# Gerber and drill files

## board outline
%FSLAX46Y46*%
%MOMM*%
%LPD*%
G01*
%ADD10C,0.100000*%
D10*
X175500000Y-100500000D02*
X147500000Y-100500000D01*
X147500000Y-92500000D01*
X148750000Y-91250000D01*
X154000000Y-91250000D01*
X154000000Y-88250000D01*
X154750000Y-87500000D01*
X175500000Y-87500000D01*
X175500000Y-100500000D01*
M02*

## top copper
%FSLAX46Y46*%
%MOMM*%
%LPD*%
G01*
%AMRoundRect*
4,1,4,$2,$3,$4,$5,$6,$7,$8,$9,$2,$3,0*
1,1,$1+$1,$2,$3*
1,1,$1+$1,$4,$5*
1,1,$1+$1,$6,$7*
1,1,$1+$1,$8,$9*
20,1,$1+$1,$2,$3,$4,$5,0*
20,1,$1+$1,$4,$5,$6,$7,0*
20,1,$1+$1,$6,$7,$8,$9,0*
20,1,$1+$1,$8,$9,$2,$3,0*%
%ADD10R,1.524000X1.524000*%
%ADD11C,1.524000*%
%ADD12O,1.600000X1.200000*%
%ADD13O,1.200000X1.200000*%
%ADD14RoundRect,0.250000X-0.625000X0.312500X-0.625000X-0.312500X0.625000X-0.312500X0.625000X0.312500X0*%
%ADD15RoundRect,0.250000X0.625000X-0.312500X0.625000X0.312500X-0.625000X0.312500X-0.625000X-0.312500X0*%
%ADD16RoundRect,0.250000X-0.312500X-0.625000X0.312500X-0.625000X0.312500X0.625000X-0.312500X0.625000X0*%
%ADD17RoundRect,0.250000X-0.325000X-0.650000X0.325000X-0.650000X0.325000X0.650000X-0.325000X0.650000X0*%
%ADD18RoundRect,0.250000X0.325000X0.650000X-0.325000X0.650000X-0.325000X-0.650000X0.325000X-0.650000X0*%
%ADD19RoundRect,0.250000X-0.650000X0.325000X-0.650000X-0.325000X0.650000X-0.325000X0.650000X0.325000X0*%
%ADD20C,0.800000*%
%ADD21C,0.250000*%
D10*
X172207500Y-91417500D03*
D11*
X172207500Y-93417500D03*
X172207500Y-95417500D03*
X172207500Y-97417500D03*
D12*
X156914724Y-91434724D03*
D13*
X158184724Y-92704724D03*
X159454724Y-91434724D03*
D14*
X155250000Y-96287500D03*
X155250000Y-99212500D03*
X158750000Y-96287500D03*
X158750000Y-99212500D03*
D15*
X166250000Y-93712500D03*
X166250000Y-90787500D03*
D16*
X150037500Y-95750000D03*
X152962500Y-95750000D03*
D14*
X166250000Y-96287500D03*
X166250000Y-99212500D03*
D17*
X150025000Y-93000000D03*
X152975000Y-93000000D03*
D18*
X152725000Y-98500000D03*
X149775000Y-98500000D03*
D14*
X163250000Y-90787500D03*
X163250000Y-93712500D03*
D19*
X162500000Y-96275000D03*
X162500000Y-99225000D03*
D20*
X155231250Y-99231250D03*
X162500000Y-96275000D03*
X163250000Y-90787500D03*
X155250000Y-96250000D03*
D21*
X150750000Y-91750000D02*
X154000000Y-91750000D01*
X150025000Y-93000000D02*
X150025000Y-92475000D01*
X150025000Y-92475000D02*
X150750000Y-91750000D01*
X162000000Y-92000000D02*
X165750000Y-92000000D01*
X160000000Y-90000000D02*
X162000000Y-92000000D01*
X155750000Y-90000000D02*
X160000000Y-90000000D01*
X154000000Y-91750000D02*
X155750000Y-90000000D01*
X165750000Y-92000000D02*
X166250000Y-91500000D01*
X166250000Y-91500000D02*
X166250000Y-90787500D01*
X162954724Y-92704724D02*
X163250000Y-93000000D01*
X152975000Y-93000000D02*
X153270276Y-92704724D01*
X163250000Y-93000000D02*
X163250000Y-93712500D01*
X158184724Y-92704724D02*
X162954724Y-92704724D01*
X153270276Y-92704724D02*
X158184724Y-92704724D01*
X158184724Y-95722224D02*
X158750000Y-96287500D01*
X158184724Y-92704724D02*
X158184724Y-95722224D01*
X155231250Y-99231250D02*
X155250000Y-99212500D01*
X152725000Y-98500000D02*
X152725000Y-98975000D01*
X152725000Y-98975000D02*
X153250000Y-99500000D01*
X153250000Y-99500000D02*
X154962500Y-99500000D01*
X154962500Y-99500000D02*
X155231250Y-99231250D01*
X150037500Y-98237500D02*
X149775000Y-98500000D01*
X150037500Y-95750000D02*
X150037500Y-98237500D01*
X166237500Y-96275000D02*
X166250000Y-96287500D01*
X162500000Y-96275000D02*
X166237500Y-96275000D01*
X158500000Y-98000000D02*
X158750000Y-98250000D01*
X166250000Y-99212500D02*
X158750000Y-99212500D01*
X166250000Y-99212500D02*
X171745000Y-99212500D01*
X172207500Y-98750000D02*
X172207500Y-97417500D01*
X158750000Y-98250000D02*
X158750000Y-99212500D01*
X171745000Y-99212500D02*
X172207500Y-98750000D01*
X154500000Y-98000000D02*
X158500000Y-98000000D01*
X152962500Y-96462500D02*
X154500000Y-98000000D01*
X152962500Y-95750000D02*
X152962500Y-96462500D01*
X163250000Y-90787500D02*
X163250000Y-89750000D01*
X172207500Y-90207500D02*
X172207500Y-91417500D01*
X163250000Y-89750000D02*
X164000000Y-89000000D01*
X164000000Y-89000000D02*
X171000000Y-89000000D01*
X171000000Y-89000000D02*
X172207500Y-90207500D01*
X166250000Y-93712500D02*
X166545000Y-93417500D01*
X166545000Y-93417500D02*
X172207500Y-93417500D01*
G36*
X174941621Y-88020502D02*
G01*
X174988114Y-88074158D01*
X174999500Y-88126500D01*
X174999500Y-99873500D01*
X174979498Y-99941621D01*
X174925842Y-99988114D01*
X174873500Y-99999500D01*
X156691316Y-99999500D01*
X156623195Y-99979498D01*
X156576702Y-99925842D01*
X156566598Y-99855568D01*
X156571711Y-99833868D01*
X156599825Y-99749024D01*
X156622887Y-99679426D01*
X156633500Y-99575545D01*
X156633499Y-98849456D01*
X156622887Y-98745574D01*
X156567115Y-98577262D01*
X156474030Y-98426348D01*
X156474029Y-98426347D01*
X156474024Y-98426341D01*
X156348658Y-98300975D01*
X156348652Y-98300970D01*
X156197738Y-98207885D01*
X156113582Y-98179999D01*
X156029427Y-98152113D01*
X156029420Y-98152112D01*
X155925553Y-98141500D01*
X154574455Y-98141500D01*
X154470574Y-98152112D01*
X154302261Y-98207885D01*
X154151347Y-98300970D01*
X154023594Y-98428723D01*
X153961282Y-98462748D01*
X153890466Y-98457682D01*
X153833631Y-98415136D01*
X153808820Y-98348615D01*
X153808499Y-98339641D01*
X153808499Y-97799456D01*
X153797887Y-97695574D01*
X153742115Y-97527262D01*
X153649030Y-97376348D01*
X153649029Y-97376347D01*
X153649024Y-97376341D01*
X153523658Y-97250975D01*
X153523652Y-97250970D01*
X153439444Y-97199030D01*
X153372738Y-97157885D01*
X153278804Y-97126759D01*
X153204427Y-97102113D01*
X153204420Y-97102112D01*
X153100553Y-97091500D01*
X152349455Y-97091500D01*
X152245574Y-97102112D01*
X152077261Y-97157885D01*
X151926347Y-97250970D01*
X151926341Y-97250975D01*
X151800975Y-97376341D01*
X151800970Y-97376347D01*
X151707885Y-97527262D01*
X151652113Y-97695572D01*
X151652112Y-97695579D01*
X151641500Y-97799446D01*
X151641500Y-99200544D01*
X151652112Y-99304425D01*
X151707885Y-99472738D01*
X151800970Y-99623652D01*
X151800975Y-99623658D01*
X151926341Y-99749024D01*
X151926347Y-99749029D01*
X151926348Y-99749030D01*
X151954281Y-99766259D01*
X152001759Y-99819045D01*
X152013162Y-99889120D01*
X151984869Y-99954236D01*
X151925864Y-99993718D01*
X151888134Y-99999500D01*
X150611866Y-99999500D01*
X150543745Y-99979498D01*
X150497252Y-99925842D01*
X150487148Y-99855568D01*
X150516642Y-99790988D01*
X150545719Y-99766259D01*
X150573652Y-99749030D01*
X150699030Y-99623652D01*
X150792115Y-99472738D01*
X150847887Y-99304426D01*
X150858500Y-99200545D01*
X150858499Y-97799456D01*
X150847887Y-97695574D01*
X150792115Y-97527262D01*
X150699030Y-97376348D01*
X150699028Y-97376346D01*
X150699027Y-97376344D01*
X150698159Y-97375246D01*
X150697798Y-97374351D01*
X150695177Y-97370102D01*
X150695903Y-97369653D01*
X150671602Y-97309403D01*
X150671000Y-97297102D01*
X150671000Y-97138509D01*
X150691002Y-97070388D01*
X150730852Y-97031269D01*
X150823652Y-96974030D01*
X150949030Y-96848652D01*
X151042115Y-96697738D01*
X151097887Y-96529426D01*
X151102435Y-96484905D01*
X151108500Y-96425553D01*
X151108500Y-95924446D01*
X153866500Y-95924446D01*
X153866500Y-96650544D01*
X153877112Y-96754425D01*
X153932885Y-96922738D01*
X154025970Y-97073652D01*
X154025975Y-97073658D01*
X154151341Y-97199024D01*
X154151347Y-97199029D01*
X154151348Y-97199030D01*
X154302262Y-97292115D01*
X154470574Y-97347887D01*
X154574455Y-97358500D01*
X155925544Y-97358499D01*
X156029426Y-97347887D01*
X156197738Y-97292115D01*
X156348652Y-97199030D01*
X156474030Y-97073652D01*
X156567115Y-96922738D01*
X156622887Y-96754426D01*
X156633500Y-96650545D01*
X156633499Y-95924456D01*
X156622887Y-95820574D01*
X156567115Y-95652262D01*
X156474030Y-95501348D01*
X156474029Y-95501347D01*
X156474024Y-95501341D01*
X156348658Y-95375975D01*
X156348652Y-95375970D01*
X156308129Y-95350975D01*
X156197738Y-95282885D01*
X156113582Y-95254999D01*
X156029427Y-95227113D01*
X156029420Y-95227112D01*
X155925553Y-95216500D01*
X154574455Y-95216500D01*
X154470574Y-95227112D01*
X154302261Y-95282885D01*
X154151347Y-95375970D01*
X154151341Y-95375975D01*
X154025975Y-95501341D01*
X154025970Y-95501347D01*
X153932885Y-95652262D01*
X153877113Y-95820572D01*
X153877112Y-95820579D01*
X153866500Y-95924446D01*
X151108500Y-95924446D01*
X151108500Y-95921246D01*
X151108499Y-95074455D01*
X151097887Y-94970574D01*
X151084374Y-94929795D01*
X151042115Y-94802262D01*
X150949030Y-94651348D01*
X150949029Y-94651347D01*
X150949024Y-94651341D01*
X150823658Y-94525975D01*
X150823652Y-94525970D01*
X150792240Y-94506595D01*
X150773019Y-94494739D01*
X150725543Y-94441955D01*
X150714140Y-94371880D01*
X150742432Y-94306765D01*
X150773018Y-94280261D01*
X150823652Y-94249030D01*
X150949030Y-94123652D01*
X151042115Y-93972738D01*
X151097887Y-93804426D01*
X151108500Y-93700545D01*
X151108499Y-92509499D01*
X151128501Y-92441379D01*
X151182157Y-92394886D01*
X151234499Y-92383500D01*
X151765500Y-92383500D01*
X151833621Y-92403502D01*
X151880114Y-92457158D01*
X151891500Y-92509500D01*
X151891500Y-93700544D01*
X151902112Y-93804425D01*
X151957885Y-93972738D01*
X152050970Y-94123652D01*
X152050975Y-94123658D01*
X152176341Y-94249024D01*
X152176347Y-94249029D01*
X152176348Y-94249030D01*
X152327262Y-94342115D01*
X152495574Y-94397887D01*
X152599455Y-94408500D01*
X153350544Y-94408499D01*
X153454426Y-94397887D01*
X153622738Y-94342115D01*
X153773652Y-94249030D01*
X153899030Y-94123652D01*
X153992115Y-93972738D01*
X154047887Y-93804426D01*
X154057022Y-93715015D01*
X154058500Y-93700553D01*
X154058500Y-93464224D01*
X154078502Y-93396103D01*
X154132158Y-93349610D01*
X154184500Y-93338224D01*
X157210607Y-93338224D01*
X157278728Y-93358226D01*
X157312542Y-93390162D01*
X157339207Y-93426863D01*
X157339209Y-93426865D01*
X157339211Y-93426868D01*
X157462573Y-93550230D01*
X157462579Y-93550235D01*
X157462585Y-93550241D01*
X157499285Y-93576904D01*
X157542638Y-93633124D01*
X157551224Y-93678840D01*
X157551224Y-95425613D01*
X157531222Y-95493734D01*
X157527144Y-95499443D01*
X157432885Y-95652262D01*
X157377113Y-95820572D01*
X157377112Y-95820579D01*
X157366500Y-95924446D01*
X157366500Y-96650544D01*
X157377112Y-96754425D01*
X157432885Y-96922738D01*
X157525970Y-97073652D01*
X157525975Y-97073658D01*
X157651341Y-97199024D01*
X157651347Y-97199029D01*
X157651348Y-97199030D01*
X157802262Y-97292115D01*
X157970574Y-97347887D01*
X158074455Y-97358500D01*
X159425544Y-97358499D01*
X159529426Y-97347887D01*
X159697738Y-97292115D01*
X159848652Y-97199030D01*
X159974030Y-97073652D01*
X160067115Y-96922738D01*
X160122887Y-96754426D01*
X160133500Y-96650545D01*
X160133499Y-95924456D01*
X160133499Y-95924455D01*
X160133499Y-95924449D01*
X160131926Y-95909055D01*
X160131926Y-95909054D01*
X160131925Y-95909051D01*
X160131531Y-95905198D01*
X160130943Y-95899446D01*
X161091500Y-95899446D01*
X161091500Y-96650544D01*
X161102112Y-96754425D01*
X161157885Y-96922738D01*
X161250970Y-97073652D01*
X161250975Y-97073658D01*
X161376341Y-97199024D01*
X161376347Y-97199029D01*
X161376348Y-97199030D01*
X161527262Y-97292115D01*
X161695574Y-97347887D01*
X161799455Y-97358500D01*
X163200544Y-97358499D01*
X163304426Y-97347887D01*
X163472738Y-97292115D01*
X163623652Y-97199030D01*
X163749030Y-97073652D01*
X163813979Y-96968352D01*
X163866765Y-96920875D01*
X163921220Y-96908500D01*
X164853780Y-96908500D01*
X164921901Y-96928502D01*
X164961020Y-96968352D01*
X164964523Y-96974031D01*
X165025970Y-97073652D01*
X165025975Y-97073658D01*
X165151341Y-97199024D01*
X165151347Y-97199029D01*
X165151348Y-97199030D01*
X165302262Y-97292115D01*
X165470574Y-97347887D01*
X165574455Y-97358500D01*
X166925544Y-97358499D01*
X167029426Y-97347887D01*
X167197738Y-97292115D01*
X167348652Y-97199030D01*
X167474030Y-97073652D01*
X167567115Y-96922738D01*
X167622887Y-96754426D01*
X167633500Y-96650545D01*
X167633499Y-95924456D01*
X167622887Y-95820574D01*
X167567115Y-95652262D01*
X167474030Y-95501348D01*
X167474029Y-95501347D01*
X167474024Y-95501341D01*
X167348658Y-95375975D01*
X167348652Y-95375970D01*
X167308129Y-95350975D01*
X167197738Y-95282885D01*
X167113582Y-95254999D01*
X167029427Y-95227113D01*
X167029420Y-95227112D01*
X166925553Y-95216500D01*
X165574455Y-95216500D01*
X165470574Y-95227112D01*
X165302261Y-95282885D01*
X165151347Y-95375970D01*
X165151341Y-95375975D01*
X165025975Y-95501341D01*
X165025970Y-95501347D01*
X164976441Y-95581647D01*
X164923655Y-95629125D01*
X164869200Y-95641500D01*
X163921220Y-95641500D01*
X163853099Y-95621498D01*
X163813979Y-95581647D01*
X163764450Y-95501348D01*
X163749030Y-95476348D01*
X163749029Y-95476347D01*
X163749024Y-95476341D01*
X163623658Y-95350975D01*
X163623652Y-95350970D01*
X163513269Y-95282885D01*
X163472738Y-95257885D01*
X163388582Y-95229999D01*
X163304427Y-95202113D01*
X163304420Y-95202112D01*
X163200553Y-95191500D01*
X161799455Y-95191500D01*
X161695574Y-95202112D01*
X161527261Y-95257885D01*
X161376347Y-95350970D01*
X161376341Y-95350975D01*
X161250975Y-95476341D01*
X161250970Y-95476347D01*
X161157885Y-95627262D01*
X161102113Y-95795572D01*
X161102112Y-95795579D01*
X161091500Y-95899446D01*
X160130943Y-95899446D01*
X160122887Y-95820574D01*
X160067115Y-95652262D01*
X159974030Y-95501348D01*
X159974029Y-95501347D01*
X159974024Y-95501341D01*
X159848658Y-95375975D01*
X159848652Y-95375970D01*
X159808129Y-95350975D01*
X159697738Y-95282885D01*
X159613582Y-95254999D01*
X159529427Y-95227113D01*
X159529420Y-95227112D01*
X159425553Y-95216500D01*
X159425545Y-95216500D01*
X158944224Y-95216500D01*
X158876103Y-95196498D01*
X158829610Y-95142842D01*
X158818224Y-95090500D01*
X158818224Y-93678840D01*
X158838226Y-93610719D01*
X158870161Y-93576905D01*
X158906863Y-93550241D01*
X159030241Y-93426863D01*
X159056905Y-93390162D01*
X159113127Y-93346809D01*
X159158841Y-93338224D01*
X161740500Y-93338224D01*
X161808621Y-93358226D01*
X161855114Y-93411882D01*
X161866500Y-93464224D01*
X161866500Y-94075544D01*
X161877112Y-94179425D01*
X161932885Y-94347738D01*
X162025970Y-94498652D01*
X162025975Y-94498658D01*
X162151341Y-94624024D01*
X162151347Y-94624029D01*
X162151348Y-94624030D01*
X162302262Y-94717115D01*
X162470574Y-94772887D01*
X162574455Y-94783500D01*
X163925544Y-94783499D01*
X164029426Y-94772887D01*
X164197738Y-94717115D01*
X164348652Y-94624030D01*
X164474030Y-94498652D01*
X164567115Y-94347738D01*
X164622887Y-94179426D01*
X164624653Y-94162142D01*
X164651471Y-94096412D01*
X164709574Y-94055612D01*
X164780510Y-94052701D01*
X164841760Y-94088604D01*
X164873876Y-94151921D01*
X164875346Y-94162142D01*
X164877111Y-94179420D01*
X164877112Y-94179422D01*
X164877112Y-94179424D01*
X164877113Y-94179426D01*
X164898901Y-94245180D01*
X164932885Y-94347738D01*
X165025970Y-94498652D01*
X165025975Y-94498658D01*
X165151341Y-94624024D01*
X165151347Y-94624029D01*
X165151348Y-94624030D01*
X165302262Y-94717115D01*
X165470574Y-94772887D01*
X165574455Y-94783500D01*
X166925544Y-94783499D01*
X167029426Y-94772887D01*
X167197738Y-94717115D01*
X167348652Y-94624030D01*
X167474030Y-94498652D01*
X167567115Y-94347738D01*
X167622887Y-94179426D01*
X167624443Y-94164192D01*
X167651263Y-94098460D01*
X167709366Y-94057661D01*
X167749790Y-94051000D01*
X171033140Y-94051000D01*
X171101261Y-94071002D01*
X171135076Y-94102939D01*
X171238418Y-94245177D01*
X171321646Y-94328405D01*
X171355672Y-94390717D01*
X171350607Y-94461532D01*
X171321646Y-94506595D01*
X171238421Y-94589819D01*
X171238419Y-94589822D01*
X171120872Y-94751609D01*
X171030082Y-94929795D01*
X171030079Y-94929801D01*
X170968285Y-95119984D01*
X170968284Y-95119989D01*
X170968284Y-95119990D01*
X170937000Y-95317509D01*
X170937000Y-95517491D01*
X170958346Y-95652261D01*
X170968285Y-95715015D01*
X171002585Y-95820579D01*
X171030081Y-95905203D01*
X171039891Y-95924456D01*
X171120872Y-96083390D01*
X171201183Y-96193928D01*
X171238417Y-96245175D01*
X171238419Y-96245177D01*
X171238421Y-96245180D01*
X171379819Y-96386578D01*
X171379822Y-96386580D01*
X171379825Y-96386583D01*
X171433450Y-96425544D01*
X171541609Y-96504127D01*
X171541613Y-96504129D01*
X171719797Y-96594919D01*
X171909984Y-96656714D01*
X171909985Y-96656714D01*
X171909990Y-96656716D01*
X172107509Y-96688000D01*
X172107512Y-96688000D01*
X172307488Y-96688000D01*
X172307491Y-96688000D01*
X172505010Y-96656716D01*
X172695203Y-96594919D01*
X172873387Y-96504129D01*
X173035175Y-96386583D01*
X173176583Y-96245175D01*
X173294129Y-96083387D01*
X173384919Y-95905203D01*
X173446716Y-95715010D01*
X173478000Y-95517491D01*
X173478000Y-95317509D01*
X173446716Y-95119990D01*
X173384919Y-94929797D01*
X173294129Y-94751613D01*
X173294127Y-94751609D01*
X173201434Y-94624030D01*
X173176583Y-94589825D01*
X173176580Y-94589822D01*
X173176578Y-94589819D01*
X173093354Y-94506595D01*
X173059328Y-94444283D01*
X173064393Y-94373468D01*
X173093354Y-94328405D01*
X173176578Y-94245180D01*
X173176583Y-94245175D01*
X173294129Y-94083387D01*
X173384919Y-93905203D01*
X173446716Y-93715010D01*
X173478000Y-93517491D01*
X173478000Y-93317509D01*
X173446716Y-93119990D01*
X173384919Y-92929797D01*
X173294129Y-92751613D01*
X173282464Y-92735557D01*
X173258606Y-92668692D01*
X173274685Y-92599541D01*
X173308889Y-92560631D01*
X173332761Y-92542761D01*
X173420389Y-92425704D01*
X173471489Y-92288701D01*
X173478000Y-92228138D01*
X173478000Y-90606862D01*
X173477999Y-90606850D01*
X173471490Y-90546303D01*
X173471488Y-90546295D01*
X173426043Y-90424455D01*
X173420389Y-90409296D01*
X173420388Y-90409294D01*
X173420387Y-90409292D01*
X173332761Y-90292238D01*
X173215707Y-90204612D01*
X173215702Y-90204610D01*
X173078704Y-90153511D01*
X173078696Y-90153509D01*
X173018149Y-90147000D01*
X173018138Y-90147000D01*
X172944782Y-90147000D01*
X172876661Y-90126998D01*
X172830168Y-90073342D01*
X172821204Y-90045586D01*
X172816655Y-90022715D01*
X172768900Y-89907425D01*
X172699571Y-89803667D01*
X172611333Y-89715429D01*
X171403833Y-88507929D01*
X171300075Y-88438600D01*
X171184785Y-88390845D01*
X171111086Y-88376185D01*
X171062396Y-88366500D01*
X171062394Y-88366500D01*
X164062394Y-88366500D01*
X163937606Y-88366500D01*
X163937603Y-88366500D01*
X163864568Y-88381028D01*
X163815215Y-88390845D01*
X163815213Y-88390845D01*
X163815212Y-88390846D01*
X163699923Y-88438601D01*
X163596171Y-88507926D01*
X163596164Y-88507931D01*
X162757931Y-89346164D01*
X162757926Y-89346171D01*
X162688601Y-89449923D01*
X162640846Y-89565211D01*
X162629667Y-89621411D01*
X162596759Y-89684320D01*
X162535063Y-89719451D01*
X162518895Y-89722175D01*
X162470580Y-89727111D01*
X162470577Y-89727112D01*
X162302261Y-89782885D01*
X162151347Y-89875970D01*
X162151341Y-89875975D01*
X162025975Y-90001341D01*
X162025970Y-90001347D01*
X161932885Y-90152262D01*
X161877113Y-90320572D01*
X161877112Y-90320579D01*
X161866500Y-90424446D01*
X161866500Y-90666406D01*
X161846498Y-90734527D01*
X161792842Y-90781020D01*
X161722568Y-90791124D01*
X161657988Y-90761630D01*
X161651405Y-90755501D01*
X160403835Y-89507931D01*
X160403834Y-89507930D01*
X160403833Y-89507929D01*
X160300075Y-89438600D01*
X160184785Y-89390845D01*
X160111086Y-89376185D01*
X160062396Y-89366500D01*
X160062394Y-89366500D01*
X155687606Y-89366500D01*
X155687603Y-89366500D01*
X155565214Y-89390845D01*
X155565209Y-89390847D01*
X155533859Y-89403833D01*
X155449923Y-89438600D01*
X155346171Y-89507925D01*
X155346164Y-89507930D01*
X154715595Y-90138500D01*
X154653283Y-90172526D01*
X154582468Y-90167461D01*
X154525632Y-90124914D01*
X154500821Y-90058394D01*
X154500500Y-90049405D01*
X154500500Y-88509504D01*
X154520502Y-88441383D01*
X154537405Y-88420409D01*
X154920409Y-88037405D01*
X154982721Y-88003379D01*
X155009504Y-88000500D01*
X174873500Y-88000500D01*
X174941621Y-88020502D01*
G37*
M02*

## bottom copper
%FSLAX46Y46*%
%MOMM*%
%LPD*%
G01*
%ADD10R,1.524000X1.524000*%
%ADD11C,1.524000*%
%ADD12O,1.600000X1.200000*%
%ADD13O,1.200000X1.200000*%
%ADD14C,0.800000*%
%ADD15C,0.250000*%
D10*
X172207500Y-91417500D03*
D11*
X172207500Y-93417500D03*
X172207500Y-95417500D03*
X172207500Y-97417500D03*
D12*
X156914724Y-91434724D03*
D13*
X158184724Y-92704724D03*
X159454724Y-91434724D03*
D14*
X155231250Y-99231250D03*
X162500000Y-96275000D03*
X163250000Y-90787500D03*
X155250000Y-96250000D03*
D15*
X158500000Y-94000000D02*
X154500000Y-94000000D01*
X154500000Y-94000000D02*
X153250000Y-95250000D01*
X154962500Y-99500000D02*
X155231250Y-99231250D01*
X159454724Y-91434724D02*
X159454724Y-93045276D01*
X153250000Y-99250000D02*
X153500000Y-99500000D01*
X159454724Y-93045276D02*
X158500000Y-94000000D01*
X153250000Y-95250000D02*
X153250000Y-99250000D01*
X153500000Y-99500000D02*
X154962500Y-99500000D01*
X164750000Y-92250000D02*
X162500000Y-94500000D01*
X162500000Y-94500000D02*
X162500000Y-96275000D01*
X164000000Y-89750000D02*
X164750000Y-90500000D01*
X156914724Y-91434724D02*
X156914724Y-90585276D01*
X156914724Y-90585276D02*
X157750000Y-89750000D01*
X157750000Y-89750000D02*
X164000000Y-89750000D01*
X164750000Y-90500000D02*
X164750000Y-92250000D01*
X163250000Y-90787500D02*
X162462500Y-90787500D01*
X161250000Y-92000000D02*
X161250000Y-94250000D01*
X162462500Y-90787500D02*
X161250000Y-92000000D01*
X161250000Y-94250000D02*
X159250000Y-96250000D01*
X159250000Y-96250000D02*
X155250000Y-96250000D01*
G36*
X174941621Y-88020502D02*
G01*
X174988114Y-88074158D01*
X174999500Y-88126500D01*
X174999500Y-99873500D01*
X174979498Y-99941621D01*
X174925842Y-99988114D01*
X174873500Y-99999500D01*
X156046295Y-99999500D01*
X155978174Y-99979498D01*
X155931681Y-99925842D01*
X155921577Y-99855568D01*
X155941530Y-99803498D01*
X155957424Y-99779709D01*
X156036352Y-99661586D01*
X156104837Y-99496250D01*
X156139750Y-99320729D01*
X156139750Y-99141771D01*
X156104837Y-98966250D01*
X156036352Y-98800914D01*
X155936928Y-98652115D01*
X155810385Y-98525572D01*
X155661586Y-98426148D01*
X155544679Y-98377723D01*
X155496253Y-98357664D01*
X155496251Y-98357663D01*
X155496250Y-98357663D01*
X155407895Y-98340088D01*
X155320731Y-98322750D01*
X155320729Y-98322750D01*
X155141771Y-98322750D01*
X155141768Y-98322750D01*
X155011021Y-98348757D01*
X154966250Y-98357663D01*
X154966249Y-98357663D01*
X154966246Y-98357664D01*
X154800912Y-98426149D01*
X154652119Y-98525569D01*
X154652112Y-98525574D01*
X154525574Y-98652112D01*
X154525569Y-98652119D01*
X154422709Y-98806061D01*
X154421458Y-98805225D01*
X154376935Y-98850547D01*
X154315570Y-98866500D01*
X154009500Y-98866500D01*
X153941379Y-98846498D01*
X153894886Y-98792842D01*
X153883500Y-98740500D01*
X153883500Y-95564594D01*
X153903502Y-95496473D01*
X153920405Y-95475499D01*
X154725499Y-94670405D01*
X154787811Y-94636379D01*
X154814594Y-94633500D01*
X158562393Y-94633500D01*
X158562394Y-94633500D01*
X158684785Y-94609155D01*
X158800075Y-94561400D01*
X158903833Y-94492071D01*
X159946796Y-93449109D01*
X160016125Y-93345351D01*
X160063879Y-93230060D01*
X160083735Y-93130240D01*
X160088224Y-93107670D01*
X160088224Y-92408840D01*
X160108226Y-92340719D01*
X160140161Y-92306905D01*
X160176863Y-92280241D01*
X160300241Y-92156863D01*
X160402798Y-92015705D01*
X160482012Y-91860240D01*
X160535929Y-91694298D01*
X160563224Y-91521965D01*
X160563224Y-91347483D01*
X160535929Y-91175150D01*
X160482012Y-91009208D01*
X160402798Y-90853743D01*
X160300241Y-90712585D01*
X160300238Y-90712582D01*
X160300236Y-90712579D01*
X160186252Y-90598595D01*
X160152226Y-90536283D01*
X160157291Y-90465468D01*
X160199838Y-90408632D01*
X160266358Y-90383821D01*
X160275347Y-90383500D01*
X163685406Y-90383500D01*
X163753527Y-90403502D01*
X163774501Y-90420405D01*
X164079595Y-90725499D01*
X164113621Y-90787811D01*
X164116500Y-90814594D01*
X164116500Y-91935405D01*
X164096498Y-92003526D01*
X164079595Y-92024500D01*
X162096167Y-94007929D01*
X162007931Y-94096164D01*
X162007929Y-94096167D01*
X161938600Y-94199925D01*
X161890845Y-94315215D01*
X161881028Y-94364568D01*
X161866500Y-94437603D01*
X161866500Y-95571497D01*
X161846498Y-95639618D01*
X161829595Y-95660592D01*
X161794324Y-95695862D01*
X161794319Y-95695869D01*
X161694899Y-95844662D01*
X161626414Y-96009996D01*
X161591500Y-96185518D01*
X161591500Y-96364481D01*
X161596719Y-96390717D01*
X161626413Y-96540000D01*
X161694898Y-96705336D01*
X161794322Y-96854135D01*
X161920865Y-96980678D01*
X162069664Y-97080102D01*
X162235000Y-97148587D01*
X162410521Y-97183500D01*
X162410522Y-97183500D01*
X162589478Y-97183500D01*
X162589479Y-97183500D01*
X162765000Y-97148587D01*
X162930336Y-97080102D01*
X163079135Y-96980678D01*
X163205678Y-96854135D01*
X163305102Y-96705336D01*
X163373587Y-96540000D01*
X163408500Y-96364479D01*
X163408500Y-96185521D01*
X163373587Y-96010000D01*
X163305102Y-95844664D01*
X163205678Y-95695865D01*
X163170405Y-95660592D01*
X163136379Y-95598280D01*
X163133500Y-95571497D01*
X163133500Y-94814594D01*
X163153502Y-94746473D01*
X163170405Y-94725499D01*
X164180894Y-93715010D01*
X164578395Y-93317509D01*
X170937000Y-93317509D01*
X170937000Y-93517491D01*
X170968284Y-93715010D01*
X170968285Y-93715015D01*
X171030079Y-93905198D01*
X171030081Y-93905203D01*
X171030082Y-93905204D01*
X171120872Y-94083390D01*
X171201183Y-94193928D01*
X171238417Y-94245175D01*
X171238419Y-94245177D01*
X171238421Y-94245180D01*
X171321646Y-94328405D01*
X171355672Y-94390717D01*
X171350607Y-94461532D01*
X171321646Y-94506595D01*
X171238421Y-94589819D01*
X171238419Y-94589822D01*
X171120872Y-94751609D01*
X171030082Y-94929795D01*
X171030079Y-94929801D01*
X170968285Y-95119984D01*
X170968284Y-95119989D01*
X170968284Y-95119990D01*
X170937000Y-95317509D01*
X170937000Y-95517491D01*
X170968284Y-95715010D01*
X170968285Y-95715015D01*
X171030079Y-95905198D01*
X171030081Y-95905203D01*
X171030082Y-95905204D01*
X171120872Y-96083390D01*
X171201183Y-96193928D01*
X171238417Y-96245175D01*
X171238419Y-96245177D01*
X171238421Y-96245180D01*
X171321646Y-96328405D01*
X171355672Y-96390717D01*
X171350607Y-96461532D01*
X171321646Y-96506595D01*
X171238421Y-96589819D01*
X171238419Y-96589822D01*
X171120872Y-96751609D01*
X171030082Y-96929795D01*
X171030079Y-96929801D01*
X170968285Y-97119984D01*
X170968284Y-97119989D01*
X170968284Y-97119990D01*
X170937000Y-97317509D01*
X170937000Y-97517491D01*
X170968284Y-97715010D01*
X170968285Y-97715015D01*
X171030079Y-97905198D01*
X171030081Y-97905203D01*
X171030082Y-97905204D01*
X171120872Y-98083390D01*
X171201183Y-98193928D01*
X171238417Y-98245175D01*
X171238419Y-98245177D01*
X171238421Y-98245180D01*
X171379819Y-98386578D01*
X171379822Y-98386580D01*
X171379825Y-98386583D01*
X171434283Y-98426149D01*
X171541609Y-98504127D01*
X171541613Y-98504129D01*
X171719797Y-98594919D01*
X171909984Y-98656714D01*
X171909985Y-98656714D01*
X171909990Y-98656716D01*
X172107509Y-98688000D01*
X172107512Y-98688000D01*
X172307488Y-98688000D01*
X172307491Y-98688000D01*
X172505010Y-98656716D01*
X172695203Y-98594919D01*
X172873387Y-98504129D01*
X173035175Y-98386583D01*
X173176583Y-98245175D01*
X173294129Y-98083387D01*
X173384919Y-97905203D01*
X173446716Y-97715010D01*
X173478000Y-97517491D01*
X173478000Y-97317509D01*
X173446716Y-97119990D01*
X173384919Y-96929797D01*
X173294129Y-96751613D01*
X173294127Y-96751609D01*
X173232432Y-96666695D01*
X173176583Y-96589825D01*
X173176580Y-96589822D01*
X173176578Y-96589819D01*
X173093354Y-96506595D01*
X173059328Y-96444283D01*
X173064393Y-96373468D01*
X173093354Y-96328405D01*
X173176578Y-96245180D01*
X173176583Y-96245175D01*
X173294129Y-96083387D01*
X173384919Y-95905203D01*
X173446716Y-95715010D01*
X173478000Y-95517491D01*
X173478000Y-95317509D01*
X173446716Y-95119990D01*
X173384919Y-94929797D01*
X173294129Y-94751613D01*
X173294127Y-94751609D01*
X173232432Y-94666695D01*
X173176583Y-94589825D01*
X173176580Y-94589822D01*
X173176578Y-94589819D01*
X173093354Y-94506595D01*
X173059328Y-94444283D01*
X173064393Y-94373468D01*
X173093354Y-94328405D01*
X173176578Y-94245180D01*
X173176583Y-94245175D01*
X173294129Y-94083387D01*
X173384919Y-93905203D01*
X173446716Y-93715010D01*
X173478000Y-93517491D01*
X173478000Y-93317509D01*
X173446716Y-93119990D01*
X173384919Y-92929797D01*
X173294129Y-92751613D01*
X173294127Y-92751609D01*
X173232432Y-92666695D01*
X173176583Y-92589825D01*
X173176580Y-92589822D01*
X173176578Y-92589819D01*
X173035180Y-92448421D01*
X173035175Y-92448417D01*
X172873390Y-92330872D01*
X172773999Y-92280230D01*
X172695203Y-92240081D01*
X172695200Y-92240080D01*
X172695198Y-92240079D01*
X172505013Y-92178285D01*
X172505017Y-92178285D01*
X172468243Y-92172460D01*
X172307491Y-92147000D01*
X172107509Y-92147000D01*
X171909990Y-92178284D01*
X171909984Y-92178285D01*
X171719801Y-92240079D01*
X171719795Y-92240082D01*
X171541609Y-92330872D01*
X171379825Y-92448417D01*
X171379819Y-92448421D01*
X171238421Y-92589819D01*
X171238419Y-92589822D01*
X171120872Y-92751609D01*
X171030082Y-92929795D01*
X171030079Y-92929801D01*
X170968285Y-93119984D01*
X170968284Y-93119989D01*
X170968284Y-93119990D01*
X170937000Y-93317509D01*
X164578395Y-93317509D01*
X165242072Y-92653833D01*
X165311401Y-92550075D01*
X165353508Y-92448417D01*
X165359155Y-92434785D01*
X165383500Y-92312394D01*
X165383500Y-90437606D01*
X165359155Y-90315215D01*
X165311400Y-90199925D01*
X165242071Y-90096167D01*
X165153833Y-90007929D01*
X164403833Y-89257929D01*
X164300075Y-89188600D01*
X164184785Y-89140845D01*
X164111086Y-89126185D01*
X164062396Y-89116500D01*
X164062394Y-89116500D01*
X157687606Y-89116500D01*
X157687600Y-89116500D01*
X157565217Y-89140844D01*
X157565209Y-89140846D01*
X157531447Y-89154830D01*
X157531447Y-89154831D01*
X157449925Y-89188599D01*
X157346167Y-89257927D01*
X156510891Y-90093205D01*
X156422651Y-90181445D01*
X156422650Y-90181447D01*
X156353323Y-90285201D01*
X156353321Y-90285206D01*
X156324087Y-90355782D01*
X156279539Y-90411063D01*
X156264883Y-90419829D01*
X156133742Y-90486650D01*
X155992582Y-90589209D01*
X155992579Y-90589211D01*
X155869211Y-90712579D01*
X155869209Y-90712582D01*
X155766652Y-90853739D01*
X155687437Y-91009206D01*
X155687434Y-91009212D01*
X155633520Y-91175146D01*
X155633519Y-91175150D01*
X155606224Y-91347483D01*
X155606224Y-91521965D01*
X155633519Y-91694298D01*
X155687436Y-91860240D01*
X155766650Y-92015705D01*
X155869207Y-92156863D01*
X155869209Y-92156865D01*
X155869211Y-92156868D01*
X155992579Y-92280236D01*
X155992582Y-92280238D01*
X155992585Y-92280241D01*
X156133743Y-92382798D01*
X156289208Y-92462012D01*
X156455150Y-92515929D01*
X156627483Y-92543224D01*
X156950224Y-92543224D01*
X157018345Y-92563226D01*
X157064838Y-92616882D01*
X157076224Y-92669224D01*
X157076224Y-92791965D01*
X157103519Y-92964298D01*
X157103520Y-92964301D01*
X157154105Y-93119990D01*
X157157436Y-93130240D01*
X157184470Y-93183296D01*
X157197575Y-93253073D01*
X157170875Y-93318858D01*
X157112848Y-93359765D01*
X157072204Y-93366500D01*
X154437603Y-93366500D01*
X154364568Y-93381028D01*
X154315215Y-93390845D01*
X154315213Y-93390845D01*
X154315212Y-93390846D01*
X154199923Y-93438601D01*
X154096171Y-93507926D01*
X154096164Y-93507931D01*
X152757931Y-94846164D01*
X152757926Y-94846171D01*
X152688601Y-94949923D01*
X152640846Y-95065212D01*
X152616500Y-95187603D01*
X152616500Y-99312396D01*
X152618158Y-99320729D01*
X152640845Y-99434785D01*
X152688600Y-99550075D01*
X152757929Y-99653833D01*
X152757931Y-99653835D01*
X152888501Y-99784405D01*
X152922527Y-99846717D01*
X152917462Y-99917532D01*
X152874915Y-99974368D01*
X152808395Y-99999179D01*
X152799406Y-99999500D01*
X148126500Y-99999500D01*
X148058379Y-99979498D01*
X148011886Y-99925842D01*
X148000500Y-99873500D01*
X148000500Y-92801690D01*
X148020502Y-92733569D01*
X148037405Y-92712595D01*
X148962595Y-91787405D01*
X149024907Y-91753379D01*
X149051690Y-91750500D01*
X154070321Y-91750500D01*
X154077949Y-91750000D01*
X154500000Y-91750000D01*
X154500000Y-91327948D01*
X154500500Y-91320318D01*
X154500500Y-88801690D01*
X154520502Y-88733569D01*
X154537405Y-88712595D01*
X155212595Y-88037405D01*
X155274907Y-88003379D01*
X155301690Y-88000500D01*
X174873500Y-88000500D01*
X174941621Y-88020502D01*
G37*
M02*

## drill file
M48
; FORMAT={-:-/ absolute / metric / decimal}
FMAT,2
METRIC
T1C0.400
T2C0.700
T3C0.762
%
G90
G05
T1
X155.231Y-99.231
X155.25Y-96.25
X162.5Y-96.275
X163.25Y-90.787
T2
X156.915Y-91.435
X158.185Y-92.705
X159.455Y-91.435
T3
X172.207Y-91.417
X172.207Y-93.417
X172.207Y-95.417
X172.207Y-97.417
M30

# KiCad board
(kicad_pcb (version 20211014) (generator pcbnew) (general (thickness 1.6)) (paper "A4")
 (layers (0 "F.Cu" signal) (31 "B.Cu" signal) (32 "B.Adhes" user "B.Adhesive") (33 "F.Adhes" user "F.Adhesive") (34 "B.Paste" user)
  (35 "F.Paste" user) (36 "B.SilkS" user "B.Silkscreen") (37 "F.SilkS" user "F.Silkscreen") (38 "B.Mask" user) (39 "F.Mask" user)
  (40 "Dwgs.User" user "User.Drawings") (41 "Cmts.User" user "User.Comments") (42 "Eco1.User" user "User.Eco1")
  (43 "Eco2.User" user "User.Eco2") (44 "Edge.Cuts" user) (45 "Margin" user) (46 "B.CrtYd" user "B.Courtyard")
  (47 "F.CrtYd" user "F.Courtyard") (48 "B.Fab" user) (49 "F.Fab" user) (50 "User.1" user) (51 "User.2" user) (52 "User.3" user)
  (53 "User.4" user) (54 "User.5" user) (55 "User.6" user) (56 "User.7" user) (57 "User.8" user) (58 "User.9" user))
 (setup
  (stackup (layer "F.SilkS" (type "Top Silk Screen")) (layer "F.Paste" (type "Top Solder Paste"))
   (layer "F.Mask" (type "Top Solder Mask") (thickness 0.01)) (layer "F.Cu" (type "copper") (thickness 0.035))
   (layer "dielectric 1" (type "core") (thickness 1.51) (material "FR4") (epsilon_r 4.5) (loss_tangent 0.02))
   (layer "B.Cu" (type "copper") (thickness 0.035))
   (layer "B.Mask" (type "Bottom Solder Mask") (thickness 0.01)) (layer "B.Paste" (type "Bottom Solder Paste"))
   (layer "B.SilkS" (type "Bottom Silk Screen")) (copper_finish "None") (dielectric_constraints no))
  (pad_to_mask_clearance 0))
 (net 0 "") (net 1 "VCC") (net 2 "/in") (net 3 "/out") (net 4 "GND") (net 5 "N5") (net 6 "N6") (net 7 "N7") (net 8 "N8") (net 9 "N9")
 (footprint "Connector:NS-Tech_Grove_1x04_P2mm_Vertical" (layer "F.Cu") (at 172.2075 91.4175)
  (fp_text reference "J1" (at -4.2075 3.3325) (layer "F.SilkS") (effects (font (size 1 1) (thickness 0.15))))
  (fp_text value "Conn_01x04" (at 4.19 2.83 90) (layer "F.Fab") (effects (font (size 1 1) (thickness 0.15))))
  (pad "1" thru_hole rect (at 0 0) (size 1.524 1.524) (drill 0.762) (layers *.Cu *.Mask) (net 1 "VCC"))
  (pad "2" thru_hole circle (at 0 2) (size 1.524 1.524) (drill 0.762) (layers *.Cu *.Mask) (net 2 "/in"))
  (pad "3" thru_hole circle (at 0 4) (size 1.524 1.524) (drill 0.762) (layers *.Cu *.Mask) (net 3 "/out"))
  (pad "4" thru_hole circle (at 0 6) (size 1.524 1.524) (drill 0.762) (layers *.Cu *.Mask) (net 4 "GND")))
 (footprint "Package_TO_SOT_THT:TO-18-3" (layer "F.Cu") (at 156.914724 91.434724)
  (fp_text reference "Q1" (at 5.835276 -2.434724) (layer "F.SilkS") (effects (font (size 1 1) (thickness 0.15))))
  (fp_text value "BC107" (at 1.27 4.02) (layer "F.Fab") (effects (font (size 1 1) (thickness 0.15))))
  (pad "1" thru_hole oval (at 0 0) (size 1.6 1.2) (drill 0.7) (layers *.Cu *.Mask) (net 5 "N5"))
  (pad "2" thru_hole oval (at 1.27 1.27) (size 1.2 1.2) (drill 0.7) (layers *.Cu *.Mask) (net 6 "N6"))
  (pad "3" thru_hole oval (at 2.54 0) (size 1.2 1.2) (drill 0.7) (layers *.Cu *.Mask) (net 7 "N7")))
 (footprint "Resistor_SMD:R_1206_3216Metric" (layer "F.Cu") (at 155.25 97.75 -90)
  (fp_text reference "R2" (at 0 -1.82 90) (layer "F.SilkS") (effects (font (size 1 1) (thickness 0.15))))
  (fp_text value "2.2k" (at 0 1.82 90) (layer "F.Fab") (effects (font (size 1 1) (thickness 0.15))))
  (pad "1" smd roundrect (at -1.4625 0 270) (size 1.125 1.75) (layers "F.Cu" "F.Paste" "F.Mask") (roundrect_rratio 0.2222222222)
   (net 1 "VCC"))
  (pad "2" smd roundrect (at 1.4625 0 270) (size 1.125 1.75) (layers "F.Cu" "F.Paste" "F.Mask") (roundrect_rratio 0.2222222222) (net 7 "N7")))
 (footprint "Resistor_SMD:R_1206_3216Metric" (layer "F.Cu") (at 158.75 97.75 -90)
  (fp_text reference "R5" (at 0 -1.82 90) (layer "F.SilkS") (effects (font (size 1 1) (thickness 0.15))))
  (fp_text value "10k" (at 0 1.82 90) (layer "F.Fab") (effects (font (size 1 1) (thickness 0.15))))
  (pad "1" smd roundrect (at -1.4625 0 270) (size 1.125 1.75) (layers "F.Cu" "F.Paste" "F.Mask") (roundrect_rratio 0.2222222222)
   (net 6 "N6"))
  (pad "2" smd roundrect (at 1.4625 0 270) (size 1.125 1.75) (layers "F.Cu" "F.Paste" "F.Mask") (roundrect_rratio 0.2222222222)
   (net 4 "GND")))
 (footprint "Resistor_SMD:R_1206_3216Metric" (layer "F.Cu") (at 166.25 92.25 90)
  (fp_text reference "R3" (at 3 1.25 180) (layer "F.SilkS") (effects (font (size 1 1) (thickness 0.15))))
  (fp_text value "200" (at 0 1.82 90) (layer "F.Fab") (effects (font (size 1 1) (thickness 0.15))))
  (pad "1" smd roundrect (at -1.4625 0 90) (size 1.125 1.75) (layers "F.Cu" "F.Paste" "F.Mask") (roundrect_rratio 0.2222222222)
   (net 2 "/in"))
  (pad "2" smd roundrect (at 1.4625 0 90) (size 1.125 1.75) (layers "F.Cu" "F.Paste" "F.Mask") (roundrect_rratio 0.2222222222) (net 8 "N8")))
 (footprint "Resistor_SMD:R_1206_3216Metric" (layer "F.Cu") (at 151.5 95.75)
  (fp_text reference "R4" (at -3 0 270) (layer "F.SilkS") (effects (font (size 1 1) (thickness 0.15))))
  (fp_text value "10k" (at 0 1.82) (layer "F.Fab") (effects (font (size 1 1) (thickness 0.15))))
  (pad "1" smd roundrect (at -1.4625 0) (size 1.125 1.75) (layers "F.Cu" "F.Paste" "F.Mask") (roundrect_rratio 0.2222222222) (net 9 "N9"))
  (pad "2" smd roundrect (at 1.4625 0) (size 1.125 1.75) (layers "F.Cu" "F.Paste" "F.Mask") (roundrect_rratio 0.2222222222) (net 4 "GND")))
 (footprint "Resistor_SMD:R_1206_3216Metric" (layer "F.Cu") (at 166.25 97.75 -90)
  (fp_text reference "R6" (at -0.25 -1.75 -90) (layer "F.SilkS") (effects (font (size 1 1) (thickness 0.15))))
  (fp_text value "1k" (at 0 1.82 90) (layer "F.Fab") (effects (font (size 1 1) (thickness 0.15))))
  (pad "1" smd roundrect (at -1.4625 0 270) (size 1.125 1.75) (layers "F.Cu" "F.Paste" "F.Mask") (roundrect_rratio 0.2222222222)
   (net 5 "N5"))
  (pad "2" smd roundrect (at 1.4625 0 270) (size 1.125 1.75) (layers "F.Cu" "F.Paste" "F.Mask") (roundrect_rratio 0.2222222222)
   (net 4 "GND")))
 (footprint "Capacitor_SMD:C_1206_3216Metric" (layer "F.Cu") (at 151.5 93)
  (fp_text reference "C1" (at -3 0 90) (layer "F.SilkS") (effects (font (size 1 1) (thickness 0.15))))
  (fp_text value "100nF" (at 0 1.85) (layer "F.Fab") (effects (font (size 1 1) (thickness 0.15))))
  (pad "1" smd roundrect (at -1.475 0) (size 1.15 1.8) (layers "F.Cu" "F.Paste" "F.Mask") (roundrect_rratio 0.2173913043) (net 8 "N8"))
  (pad "2" smd roundrect (at 1.475 0) (size 1.15 1.8) (layers "F.Cu" "F.Paste" "F.Mask") (roundrect_rratio 0.2173913043) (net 6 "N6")))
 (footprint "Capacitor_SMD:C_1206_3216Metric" (layer "F.Cu") (at 151.25 98.5 180)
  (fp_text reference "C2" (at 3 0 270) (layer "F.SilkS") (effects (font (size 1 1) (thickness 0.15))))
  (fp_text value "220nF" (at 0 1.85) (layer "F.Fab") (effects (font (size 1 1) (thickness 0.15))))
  (pad "1" smd roundrect (at -1.475 0 180) (size 1.15 1.8) (layers "F.Cu" "F.Paste" "F.Mask") (roundrect_rratio 0.2173913043) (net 7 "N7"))
  (pad "2" smd roundrect (at 1.475 0 180) (size 1.15 1.8) (layers "F.Cu" "F.Paste" "F.Mask") (roundrect_rratio 0.2173913043) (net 9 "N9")))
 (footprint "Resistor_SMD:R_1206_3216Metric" (layer "F.Cu") (at 163.25 92.25 -90)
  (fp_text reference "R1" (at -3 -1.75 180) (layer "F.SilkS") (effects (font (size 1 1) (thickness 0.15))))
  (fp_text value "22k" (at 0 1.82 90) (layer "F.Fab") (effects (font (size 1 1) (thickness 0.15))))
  (pad "1" smd roundrect (at -1.4625 0 270) (size 1.125 1.75) (layers "F.Cu" "F.Paste" "F.Mask") (roundrect_rratio 0.2222222222)
   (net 1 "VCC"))
  (pad "2" smd roundrect (at 1.4625 0 270) (size 1.125 1.75) (layers "F.Cu" "F.Paste" "F.Mask") (roundrect_rratio 0.2222222222) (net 6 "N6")))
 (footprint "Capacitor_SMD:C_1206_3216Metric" (layer "F.Cu") (at 162.5 97.75 -90)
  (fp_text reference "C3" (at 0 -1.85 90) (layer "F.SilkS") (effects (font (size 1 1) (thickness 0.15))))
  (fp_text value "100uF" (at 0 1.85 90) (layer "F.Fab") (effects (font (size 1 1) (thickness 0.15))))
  (pad "1" smd roundrect (at -1.475 0 270) (size 1.15 1.8) (layers "F.Cu" "F.Paste" "F.Mask") (roundrect_rratio 0.2173913043) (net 5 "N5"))
  (pad "2" smd roundrect (at 1.475 0 270) (size 1.15 1.8) (layers "F.Cu" "F.Paste" "F.Mask") (roundrect_rratio 0.2173913043) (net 4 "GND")))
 (gr_poly
  (pts (xy 175.5 100.5) (xy 147.5 100.5) (xy 147.5 92.5) (xy 148.75 91.25) (xy 154 91.25) (xy 154 88.25) (xy 154.75 87.5) (xy 175.5 87.5))
  (layer "Edge.Cuts") (width 0.1) (fill none))
 (segment (start 150.75 91.75) (end 154 91.75) (width 0.25) (layer "F.Cu") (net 8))
 (segment (start 150.025 93) (end 150.025 92.475) (width 0.25) (layer "F.Cu") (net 8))
 (segment (start 150.025 92.475) (end 150.75 91.75) (width 0.25) (layer "F.Cu") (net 8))
 (segment (start 162 92) (end 165.75 92) (width 0.25) (layer "F.Cu") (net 8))
 (segment (start 160 90) (end 162 92) (width 0.25) (layer "F.Cu") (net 8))
 (segment (start 155.75 90) (end 160 90) (width 0.25) (layer "F.Cu") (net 8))
 (segment (start 154 91.75) (end 155.75 90) (width 0.25) (layer "F.Cu") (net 8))
 (segment (start 165.75 92) (end 166.25 91.5) (width 0.25) (layer "F.Cu") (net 8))
 (segment (start 166.25 91.5) (end 166.25 90.7875) (width 0.25) (layer "F.Cu") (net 8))
 (segment (start 162.954724 92.704724) (end 163.25 93) (width 0.25) (layer "F.Cu") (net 6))
 (segment (start 152.975 93) (end 153.270276 92.704724) (width 0.25) (layer "F.Cu") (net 6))
 (segment (start 163.25 93) (end 163.25 93.7125) (width 0.25) (layer "F.Cu") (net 6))
 (segment (start 158.184724 92.704724) (end 162.954724 92.704724) (width 0.25) (layer "F.Cu") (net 6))
 (segment (start 153.270276 92.704724) (end 158.184724 92.704724) (width 0.25) (layer "F.Cu") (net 6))
 (segment (start 158.184724 95.722224) (end 158.75 96.2875) (width 0.25) (layer "F.Cu") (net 6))
 (segment (start 158.184724 92.704724) (end 158.184724 95.722224) (width 0.25) (layer "F.Cu") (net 6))
 (segment (start 155.23125 99.23125) (end 155.25 99.2125) (width 0.25) (layer "F.Cu") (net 7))
 (segment (start 152.725 98.5) (end 152.725 98.975) (width 0.25) (layer "F.Cu") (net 7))
 (segment (start 152.725 98.975) (end 153.25 99.5) (width 0.25) (layer "F.Cu") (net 7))
 (segment (start 153.25 99.5) (end 154.9625 99.5) (width 0.25) (layer "F.Cu") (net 7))
 (segment (start 154.9625 99.5) (end 155.23125 99.23125) (width 0.25) (layer "F.Cu") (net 7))
 (via (at 155.23125 99.23125) (size 0.8) (drill 0.4) (layers "F.Cu" "B.Cu") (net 7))
 (segment (start 158.5 94) (end 154.5 94) (width 0.25) (layer "B.Cu") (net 7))
 (segment (start 154.5 94) (end 153.25 95.25) (width 0.25) (layer "B.Cu") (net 7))
 (segment (start 154.9625 99.5) (end 155.23125 99.23125) (width 0.25) (layer "B.Cu") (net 7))
 (segment (start 159.454724 91.434724) (end 159.454724 93.045276) (width 0.25) (layer "B.Cu") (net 7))
 (segment (start 153.25 99.25) (end 153.5 99.5) (width 0.25) (layer "B.Cu") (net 7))
 (segment (start 159.454724 93.045276) (end 158.5 94) (width 0.25) (layer "B.Cu") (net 7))
 (segment (start 153.25 95.25) (end 153.25 99.25) (width 0.25) (layer "B.Cu") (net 7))
 (segment (start 153.5 99.5) (end 154.9625 99.5) (width 0.25) (layer "B.Cu") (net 7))
 (segment (start 150.0375 98.2375) (end 149.775 98.5) (width 0.25) (layer "F.Cu") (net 9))
 (segment (start 150.0375 95.75) (end 150.0375 98.2375) (width 0.25) (layer "F.Cu") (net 9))
 (segment (start 166.2375 96.275) (end 166.25 96.2875) (width 0.25) (layer "F.Cu") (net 5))
 (segment (start 162.5 96.275) (end 166.2375 96.275) (width 0.25) (layer "F.Cu") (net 5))
 (via (at 162.5 96.275) (size 0.8) (drill 0.4) (layers "F.Cu" "B.Cu") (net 5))
 (segment (start 164.75 92.25) (end 162.5 94.5) (width 0.25) (layer "B.Cu") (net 5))
 (segment (start 162.5 94.5) (end 162.5 96.275) (width 0.25) (layer "B.Cu") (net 5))
 (segment (start 164 89.75) (end 164.75 90.5) (width 0.25) (layer "B.Cu") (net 5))
 (segment (start 156.914724 91.434724) (end 156.914724 90.585276) (width 0.25) (layer "B.Cu") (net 5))
 (segment (start 156.914724 90.585276) (end 157.75 89.75) (width 0.25) (layer "B.Cu") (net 5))
 (segment (start 157.75 89.75) (end 164 89.75) (width 0.25) (layer "B.Cu") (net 5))
 (segment (start 164.75 90.5) (end 164.75 92.25) (width 0.25) (layer "B.Cu") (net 5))
 (segment (start 158.5 98) (end 158.75 98.25) (width 0.25) (layer "F.Cu") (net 4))
 (segment (start 166.25 99.2125) (end 158.75 99.2125) (width 0.25) (layer "F.Cu") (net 4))
 (segment (start 166.25 99.2125) (end 171.745 99.2125) (width 0.25) (layer "F.Cu") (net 4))
 (segment (start 172.2075 98.75) (end 172.2075 97.4175) (width 0.25) (layer "F.Cu") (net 4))
 (segment (start 158.75 98.25) (end 158.75 99.2125) (width 0.25) (layer "F.Cu") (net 4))
 (segment (start 171.745 99.2125) (end 172.2075 98.75) (width 0.25) (layer "F.Cu") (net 4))
 (segment (start 154.5 98) (end 158.5 98) (width 0.25) (layer "F.Cu") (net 4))
 (segment (start 152.9625 96.4625) (end 154.5 98) (width 0.25) (layer "F.Cu") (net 4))
 (segment (start 152.9625 95.75) (end 152.9625 96.4625) (width 0.25) (layer "F.Cu") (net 4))
 (segment (start 163.25 90.7875) (end 163.25 89.75) (width 0.25) (layer "F.Cu") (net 1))
 (segment (start 172.2075 90.2075) (end 172.2075 91.4175) (width 0.25) (layer "F.Cu") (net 1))
 (segment (start 163.25 89.75) (end 164 89) (width 0.25) (layer "F.Cu") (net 1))
 (segment (start 164 89) (end 171 89) (width 0.25) (layer "F.Cu") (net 1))
 (segment (start 171 89) (end 172.2075 90.2075) (width 0.25) (layer "F.Cu") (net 1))
 (via (at 163.25 90.7875) (size 0.8) (drill 0.4) (layers "F.Cu" "B.Cu") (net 1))
 (via (at 155.25 96.25) (size 0.8) (drill 0.4) (layers "F.Cu" "B.Cu") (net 1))
 (segment (start 163.25 90.7875) (end 162.4625 90.7875) (width 0.25) (layer "B.Cu") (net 1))
 (segment (start 161.25 92) (end 161.25 94.25) (width 0.25) (layer "B.Cu") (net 1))
 (segment (start 162.4625 90.7875) (end 161.25 92) (width 0.25) (layer "B.Cu") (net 1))
 (segment (start 161.25 94.25) (end 159.25 96.25) (width 0.25) (layer "B.Cu") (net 1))
 (segment (start 159.25 96.25) (end 155.25 96.25) (width 0.25) (layer "B.Cu") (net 1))
 (segment (start 166.25 93.7125) (end 166.545 93.4175) (width 0.25) (layer "F.Cu") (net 2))
 (segment (start 166.545 93.4175) (end 172.2075 93.4175) (width 0.25) (layer "F.Cu") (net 2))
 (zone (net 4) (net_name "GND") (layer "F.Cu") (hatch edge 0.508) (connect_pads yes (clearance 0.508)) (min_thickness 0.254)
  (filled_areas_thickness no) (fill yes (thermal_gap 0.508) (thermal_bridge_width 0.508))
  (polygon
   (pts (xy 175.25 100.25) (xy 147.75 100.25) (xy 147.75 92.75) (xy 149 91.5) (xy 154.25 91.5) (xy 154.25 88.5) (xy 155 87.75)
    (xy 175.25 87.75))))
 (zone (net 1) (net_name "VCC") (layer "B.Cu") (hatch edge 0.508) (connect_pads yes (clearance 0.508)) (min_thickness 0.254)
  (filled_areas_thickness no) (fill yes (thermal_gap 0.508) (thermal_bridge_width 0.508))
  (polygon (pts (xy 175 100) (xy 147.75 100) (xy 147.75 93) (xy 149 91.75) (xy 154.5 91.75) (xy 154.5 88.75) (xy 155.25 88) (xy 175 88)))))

